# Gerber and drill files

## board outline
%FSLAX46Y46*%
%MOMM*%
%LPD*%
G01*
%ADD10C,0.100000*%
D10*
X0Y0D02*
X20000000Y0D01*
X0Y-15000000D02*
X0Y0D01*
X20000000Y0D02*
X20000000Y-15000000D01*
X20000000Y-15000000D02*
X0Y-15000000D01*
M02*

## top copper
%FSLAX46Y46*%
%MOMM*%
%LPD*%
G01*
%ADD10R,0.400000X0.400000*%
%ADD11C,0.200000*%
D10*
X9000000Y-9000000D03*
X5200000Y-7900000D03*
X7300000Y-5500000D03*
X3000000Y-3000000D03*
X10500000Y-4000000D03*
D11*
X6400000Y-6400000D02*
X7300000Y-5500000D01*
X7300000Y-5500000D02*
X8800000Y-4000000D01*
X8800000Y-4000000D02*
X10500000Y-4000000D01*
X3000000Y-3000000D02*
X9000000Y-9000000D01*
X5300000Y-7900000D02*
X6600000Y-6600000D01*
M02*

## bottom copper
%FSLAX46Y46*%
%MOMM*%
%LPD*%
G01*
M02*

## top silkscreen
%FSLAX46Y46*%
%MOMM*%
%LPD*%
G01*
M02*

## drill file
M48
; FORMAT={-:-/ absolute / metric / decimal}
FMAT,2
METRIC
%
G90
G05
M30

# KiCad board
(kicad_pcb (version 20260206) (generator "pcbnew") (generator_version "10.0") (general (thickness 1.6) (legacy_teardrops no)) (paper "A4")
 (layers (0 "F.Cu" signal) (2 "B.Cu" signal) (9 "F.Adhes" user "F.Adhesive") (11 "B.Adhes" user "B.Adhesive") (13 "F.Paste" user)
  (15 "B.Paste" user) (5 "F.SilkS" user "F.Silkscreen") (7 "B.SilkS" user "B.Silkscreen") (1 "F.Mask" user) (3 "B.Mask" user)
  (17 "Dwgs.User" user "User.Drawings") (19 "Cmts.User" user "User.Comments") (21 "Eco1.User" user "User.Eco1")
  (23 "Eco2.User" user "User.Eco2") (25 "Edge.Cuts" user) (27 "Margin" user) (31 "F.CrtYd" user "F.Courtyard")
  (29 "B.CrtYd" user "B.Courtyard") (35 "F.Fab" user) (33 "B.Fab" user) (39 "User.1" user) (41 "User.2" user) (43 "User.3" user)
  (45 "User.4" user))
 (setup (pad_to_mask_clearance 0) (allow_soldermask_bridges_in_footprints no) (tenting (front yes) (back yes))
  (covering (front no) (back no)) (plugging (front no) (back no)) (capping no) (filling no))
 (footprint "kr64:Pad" (layer "F.Cu") (at 9 9)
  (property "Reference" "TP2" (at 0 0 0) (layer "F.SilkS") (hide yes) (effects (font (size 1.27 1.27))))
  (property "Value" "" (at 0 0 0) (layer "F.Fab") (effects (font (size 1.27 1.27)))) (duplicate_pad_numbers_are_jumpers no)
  (pad "1" smd rect (at 0 0) (size 0.4 0.4) (layers "F.Cu" "F.Mask" "F.Paste") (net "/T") (thermal_bridge_angle 45)))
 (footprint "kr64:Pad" (layer "F.Cu") (at 5.2 7.9)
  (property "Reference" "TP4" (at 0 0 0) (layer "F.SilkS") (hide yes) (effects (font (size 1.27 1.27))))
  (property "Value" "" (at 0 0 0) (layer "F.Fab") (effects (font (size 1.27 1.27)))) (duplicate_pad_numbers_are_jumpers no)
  (pad "1" smd rect (at 0 0) (size 0.4 0.4) (layers "F.Cu" "F.Mask" "F.Paste") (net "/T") (thermal_bridge_angle 45)))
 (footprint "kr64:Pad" (layer "F.Cu") (at 7.3 5.5)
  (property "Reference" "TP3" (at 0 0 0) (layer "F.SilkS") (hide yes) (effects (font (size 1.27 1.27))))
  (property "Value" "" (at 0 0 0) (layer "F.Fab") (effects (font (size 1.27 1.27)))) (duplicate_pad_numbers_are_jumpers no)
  (pad "1" smd rect (at 0 0) (size 0.4 0.4) (layers "F.Cu" "F.Mask" "F.Paste") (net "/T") (thermal_bridge_angle 45)))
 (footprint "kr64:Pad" (layer "F.Cu") (at 3 3)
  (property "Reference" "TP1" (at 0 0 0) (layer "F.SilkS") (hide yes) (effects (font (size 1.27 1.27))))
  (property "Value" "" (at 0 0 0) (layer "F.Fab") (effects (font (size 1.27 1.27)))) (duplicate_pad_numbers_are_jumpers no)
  (pad "1" smd rect (at 0 0) (size 0.4 0.4) (layers "F.Cu" "F.Mask" "F.Paste") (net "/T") (thermal_bridge_angle 45)))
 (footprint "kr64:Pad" (layer "F.Cu") (at 10.5 4)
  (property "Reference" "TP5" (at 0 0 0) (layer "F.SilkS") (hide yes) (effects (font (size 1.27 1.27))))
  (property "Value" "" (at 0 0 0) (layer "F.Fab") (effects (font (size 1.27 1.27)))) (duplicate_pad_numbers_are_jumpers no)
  (pad "1" smd rect (at 0 0) (size 0.4 0.4) (layers "F.Cu" "F.Mask" "F.Paste") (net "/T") (thermal_bridge_angle 45)))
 (gr_line (start 0 0) (end 20 0) (stroke (width 0.1) (type default)) (layer "Edge.Cuts"))
 (gr_line (start 0 15) (end 0 0) (stroke (width 0.1) (type default)) (layer "Edge.Cuts"))
 (gr_line (start 20 0) (end 20 15) (stroke (width 0.1) (type default)) (layer "Edge.Cuts"))
 (gr_line (start 20 15) (end 0 15) (stroke (width 0.1) (type default)) (layer "Edge.Cuts"))
 (segment (start 6.4 6.4) (end 7.3 5.5) (width 0.2) (layer "F.Cu") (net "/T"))
 (segment (start 7.3 5.5) (end 8.8 4) (width 0.2) (layer "F.Cu") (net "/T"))
 (segment (start 8.8 4) (end 10.5 4) (width 0.2) (layer "F.Cu") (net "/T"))
 (segment (start 3 3) (end 9 9) (width 0.2) (layer "F.Cu") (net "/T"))
 (segment (start 5.3 7.9) (end 6.6 6.6) (width 0.2) (layer "F.Cu") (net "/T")))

